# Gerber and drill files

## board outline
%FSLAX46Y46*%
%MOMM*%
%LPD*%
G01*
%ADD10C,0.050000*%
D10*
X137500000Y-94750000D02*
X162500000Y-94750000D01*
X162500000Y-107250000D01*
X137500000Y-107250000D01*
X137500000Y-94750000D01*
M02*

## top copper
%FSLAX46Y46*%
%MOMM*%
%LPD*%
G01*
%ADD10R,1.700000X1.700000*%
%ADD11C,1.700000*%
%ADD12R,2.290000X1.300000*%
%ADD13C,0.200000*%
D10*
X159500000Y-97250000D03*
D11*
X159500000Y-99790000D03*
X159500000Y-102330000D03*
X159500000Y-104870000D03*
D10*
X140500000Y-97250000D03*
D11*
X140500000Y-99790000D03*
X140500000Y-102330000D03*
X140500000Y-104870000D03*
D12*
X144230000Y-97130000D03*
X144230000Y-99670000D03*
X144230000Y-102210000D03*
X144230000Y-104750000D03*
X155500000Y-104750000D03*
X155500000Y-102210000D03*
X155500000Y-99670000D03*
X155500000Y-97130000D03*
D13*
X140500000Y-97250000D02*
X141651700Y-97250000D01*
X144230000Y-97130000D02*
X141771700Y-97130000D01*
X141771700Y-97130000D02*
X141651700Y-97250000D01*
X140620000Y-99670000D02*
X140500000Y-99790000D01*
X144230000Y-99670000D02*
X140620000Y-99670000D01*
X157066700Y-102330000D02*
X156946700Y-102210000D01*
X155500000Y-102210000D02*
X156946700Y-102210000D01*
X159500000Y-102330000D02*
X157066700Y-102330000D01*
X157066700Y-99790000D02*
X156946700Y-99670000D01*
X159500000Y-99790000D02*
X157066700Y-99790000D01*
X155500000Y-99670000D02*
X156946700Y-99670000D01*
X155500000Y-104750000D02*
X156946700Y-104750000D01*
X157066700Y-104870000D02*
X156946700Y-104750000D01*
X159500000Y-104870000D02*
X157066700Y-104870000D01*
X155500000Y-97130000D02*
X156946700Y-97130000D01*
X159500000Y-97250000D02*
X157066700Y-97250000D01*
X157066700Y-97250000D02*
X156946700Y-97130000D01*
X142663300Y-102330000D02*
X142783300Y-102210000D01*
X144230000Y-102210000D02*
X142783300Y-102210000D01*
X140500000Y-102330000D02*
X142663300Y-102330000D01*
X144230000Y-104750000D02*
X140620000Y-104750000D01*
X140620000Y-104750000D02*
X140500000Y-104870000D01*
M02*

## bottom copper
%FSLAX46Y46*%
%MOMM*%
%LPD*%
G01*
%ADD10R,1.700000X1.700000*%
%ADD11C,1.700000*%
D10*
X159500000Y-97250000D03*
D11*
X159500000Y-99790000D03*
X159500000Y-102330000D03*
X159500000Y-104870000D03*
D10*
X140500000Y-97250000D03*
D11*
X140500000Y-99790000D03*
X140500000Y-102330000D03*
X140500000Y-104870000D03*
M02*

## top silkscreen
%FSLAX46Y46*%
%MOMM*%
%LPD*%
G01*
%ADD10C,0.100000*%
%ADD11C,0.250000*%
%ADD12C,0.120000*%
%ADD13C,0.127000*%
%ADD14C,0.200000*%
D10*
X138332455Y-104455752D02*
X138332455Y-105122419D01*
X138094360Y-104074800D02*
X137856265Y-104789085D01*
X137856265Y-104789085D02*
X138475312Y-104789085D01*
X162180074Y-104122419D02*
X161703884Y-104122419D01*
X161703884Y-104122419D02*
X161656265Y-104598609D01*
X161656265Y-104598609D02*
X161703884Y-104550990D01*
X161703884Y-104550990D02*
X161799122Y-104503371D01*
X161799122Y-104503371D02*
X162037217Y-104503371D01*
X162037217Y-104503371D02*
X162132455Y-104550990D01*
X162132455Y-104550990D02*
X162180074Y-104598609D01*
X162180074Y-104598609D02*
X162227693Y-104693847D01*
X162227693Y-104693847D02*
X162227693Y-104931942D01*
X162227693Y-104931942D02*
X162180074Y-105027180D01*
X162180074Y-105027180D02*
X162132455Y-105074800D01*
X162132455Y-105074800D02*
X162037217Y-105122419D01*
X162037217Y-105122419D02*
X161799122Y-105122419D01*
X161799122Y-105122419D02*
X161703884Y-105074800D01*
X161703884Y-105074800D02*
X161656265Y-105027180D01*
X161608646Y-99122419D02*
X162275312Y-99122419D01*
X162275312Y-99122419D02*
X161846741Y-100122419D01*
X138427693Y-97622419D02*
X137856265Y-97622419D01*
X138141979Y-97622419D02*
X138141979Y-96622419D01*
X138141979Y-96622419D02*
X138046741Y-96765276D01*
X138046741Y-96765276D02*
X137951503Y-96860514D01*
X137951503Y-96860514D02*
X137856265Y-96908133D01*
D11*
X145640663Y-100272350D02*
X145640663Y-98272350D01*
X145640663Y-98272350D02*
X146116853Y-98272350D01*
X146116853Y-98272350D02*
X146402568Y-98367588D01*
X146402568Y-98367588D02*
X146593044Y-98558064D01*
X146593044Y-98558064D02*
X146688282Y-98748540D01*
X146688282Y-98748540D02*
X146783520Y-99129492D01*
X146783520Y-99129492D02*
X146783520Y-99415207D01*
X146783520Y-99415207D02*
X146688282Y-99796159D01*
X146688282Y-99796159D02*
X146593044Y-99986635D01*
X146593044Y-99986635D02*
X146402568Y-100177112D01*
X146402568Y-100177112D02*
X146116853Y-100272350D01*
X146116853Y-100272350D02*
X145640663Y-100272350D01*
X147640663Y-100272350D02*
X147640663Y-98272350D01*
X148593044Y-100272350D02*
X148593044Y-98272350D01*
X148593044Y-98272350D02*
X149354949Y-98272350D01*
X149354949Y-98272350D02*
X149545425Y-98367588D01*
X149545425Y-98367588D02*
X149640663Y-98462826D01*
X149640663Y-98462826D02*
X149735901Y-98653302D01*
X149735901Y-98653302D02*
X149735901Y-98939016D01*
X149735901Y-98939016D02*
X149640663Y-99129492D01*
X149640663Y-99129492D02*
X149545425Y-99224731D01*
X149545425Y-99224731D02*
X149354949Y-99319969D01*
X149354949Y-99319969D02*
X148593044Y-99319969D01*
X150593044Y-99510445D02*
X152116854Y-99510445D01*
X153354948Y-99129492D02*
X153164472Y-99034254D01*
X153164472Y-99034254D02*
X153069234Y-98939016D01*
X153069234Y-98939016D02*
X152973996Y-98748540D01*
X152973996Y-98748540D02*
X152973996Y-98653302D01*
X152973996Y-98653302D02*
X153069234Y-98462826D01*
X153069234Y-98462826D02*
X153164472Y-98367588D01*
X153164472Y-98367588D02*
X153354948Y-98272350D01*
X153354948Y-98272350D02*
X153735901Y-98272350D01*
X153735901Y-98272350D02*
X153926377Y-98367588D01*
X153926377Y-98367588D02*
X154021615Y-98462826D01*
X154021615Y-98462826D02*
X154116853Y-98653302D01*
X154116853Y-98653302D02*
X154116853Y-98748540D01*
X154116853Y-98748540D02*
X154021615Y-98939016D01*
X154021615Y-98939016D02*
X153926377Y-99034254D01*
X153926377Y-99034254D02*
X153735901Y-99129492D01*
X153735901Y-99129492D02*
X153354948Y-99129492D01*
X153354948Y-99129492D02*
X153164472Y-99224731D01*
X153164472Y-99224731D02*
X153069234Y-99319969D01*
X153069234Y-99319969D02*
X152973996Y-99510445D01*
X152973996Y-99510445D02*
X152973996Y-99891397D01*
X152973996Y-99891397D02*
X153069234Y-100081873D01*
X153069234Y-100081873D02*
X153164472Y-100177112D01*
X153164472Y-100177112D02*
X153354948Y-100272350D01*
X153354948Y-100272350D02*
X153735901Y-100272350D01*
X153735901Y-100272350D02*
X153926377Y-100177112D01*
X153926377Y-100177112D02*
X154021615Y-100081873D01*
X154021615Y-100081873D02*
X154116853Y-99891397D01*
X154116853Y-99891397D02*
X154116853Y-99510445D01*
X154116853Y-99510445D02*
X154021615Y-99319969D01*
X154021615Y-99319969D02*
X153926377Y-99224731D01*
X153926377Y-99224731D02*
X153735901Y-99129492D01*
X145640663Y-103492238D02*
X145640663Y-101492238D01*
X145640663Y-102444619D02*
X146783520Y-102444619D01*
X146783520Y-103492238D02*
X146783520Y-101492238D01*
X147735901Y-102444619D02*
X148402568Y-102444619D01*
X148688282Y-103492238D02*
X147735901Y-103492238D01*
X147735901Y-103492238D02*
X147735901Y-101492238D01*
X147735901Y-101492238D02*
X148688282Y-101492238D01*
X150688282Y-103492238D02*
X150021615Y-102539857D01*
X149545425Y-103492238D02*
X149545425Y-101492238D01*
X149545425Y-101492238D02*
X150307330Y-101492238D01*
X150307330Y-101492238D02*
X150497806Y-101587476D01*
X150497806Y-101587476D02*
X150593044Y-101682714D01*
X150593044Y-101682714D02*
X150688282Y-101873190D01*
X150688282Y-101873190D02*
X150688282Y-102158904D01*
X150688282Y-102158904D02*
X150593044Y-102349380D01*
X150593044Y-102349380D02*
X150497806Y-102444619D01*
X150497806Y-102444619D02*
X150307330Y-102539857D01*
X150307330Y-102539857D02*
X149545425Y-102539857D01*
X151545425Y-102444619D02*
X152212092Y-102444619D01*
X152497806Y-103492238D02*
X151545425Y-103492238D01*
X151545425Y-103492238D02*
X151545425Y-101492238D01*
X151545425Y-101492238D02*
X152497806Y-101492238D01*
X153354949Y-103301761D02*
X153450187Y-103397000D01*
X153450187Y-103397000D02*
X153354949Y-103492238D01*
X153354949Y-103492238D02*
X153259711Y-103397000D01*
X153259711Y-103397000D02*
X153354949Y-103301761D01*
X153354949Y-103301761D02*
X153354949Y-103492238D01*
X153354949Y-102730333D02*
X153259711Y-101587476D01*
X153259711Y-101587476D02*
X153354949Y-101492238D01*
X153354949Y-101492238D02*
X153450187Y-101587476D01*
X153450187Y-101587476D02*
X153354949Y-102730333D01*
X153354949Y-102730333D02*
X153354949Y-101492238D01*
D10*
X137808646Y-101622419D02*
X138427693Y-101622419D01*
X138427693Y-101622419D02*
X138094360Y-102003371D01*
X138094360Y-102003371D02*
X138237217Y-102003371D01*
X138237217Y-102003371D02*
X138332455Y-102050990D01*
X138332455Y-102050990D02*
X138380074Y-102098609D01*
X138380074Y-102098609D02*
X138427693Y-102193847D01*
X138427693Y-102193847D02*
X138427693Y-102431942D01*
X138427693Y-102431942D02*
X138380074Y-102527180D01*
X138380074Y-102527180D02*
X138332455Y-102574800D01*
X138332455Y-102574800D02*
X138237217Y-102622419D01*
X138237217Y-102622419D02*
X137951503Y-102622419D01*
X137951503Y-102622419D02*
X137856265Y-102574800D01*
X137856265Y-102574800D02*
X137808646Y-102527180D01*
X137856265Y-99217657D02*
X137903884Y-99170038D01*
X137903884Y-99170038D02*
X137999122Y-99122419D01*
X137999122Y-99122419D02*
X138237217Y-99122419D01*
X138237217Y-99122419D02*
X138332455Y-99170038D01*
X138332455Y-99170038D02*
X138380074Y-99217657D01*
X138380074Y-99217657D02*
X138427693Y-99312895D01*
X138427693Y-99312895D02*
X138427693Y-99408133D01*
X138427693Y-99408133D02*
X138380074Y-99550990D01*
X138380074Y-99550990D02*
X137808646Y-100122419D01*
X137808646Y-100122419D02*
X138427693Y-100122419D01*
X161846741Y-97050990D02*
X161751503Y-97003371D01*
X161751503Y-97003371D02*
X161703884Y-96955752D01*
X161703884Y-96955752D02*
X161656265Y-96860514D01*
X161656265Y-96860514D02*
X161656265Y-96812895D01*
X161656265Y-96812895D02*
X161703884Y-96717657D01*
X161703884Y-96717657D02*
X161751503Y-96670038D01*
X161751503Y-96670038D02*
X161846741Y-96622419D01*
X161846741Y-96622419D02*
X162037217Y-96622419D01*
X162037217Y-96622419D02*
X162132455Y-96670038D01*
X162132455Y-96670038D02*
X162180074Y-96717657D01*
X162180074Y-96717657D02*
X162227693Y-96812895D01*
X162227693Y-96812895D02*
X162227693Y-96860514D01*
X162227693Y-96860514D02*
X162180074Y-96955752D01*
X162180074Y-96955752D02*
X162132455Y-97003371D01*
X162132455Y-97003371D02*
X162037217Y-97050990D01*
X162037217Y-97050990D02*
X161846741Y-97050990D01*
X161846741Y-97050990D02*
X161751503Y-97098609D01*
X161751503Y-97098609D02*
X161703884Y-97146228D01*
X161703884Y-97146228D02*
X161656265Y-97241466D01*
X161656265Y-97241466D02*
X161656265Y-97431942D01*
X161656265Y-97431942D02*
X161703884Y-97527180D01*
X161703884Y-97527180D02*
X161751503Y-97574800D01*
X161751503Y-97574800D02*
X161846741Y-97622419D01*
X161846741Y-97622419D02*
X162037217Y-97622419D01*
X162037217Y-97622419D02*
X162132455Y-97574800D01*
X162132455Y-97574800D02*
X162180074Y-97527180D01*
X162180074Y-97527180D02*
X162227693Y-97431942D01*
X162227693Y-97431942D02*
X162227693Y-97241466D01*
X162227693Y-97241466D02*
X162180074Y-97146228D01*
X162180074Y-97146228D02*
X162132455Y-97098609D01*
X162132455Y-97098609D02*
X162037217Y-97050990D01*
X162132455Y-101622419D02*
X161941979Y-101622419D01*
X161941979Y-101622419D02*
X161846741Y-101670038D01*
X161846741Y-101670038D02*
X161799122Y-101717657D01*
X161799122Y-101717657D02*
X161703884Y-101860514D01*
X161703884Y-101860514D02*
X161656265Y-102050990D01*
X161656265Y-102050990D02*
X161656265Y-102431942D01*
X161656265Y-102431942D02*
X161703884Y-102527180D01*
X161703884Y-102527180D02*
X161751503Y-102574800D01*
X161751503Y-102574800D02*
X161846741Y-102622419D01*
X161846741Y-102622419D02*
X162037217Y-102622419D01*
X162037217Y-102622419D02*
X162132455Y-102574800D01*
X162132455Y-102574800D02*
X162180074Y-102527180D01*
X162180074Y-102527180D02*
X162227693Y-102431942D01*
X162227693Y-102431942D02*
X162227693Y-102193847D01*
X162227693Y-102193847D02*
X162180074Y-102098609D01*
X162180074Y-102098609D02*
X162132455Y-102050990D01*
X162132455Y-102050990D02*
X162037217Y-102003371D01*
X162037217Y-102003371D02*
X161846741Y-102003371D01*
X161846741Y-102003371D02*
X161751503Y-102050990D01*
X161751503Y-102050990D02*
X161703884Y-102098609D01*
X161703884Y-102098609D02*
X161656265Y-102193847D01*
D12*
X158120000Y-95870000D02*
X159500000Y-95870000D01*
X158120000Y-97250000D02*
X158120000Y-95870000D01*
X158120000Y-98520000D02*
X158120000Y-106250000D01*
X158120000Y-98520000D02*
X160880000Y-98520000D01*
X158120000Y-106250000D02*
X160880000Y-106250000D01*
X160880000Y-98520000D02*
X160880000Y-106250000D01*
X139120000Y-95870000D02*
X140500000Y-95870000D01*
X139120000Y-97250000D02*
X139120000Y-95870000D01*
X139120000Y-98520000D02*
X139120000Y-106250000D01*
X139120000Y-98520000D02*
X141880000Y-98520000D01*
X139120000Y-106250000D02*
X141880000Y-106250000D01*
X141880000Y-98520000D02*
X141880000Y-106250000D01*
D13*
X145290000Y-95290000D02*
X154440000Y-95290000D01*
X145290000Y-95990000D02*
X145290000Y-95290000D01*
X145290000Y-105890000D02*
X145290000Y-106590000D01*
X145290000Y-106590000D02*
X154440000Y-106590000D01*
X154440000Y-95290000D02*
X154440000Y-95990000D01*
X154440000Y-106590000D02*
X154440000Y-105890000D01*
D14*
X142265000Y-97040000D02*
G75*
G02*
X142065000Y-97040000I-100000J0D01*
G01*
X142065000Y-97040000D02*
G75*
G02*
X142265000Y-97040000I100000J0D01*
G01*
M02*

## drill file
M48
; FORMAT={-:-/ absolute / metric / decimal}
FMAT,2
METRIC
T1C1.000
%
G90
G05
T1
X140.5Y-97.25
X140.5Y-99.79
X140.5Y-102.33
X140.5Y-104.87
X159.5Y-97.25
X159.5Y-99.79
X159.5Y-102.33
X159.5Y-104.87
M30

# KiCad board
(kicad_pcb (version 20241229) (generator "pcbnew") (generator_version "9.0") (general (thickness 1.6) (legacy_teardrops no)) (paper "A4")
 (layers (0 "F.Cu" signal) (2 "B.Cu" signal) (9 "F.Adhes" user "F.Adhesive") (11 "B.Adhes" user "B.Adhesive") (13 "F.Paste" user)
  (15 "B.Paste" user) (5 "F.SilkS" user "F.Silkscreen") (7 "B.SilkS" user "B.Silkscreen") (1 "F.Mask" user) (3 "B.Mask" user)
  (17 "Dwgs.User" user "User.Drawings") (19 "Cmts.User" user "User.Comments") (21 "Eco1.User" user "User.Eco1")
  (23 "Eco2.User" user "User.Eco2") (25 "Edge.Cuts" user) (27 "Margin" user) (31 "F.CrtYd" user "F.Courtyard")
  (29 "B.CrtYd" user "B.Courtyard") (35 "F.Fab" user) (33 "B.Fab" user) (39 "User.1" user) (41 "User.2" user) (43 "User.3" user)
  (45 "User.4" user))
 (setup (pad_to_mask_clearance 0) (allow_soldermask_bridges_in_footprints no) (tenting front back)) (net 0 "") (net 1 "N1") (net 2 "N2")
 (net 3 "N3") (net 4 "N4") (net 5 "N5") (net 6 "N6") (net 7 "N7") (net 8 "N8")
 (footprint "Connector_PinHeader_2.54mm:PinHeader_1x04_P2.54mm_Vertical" (layer "F.Cu") (at 159.5 97.25)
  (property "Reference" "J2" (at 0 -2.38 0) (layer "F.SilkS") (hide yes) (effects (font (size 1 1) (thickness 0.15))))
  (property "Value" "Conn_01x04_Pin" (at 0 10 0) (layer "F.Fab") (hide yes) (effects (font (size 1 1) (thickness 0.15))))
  (fp_line (start -1.38 -1.38) (end 0 -1.38) (stroke (width 0.12) (type solid)) (layer "F.SilkS"))
  (fp_line (start -1.38 0) (end -1.38 -1.38) (stroke (width 0.12) (type solid)) (layer "F.SilkS"))
  (fp_line (start -1.38 1.27) (end -1.38 9) (stroke (width 0.12) (type solid)) (layer "F.SilkS"))
  (fp_line (start -1.38 1.27) (end 1.38 1.27) (stroke (width 0.12) (type solid)) (layer "F.SilkS"))
  (fp_line (start -1.38 9) (end 1.38 9) (stroke (width 0.12) (type solid)) (layer "F.SilkS"))
  (fp_line (start 1.38 1.27) (end 1.38 9) (stroke (width 0.12) (type solid)) (layer "F.SilkS"))
  (pad "1" thru_hole rect (at 0 0) (size 1.7 1.7) (drill 1) (layers "*.Cu" "*.Mask") (remove_unused_layers no) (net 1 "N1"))
  (pad "2" thru_hole circle (at 0 2.54) (size 1.7 1.7) (drill 1) (layers "*.Cu" "*.Mask") (remove_unused_layers no) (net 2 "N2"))
  (pad "3" thru_hole circle (at 0 5.08) (size 1.7 1.7) (drill 1) (layers "*.Cu" "*.Mask") (remove_unused_layers no) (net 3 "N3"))
  (pad "4" thru_hole circle (at 0 7.62) (size 1.7 1.7) (drill 1) (layers "*.Cu" "*.Mask") (remove_unused_layers no) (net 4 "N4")))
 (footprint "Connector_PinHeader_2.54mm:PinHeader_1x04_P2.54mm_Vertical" (layer "F.Cu") (at 140.5 97.25)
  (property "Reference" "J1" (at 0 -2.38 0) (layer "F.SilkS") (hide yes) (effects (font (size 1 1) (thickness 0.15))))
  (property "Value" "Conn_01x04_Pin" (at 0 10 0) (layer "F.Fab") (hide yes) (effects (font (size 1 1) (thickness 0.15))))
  (fp_line (start -1.38 -1.38) (end 0 -1.38) (stroke (width 0.12) (type solid)) (layer "F.SilkS"))
  (fp_line (start -1.38 0) (end -1.38 -1.38) (stroke (width 0.12) (type solid)) (layer "F.SilkS"))
  (fp_line (start -1.38 1.27) (end -1.38 9) (stroke (width 0.12) (type solid)) (layer "F.SilkS"))
  (fp_line (start -1.38 1.27) (end 1.38 1.27) (stroke (width 0.12) (type solid)) (layer "F.SilkS"))
  (fp_line (start -1.38 9) (end 1.38 9) (stroke (width 0.12) (type solid)) (layer "F.SilkS"))
  (fp_line (start 1.38 1.27) (end 1.38 9) (stroke (width 0.12) (type solid)) (layer "F.SilkS"))
  (pad "1" thru_hole rect (at 0 0) (size 1.7 1.7) (drill 1) (layers "*.Cu" "*.Mask") (remove_unused_layers no) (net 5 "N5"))
  (pad "2" thru_hole circle (at 0 2.54) (size 1.7 1.7) (drill 1) (layers "*.Cu" "*.Mask") (remove_unused_layers no) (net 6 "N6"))
  (pad "3" thru_hole circle (at 0 5.08) (size 1.7 1.7) (drill 1) (layers "*.Cu" "*.Mask") (remove_unused_layers no) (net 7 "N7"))
  (pad "4" thru_hole circle (at 0 7.62) (size 1.7 1.7) (drill 1) (layers "*.Cu" "*.Mask") (remove_unused_layers no) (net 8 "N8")))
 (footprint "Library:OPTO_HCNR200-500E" (layer "F.Cu") (at 149.865 100.94)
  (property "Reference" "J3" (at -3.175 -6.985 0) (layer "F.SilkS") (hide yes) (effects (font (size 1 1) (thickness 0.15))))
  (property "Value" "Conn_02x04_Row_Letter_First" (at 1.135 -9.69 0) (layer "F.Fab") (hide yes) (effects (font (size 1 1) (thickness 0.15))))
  (fp_line (start -4.575 -5.65) (end 4.575 -5.65) (stroke (width 0.127) (type solid)) (layer "F.SilkS"))
  (fp_line (start -4.575 -4.95) (end -4.575 -5.65) (stroke (width 0.127) (type solid)) (layer "F.SilkS"))
  (fp_line (start -4.575 4.95) (end -4.575 5.65) (stroke (width 0.127) (type solid)) (layer "F.SilkS"))
  (fp_line (start -4.575 5.65) (end 4.575 5.65) (stroke (width 0.127) (type solid)) (layer "F.SilkS"))
  (fp_line (start 4.575 -5.65) (end 4.575 -4.95) (stroke (width 0.127) (type solid)) (layer "F.SilkS"))
  (fp_line (start 4.575 5.65) (end 4.575 4.95) (stroke (width 0.127) (type solid)) (layer "F.SilkS"))
  (fp_circle (center -7.7 -3.9) (end -7.6 -3.9) (stroke (width 0.2) (type solid)) (fill no) (layer "F.SilkS"))
  (pad "1" smd rect (at -5.635 -3.81) (size 2.29 1.3) (layers "F.Cu" "F.Mask" "F.Paste") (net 5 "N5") (solder_mask_margin 0.102))
  (pad "2" smd rect (at -5.635 -1.27) (size 2.29 1.3) (layers "F.Cu" "F.Mask" "F.Paste") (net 6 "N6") (solder_mask_margin 0.102))
  (pad "3" smd rect (at -5.635 1.27) (size 2.29 1.3) (layers "F.Cu" "F.Mask" "F.Paste") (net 7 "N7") (solder_mask_margin 0.102))
  (pad "4" smd rect (at -5.635 3.81) (size 2.29 1.3) (layers "F.Cu" "F.Mask" "F.Paste") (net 8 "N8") (solder_mask_margin 0.102))
  (pad "5" smd rect (at 5.635 3.81) (size 2.29 1.3) (layers "F.Cu" "F.Mask" "F.Paste") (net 4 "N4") (solder_mask_margin 0.102))
  (pad "6" smd rect (at 5.635 1.27) (size 2.29 1.3) (layers "F.Cu" "F.Mask" "F.Paste") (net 3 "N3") (solder_mask_margin 0.102))
  (pad "7" smd rect (at 5.635 -1.27) (size 2.29 1.3) (layers "F.Cu" "F.Mask" "F.Paste") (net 2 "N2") (solder_mask_margin 0.102))
  (pad "8" smd rect (at 5.635 -3.81) (size 2.29 1.3) (layers "F.Cu" "F.Mask" "F.Paste") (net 1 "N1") (solder_mask_margin 0.102)))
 (gr_rect (start 137.5 94.75) (end 162.5 107.25) (stroke (width 0.05) (type default)) (fill no) (layer "Edge.Cuts"))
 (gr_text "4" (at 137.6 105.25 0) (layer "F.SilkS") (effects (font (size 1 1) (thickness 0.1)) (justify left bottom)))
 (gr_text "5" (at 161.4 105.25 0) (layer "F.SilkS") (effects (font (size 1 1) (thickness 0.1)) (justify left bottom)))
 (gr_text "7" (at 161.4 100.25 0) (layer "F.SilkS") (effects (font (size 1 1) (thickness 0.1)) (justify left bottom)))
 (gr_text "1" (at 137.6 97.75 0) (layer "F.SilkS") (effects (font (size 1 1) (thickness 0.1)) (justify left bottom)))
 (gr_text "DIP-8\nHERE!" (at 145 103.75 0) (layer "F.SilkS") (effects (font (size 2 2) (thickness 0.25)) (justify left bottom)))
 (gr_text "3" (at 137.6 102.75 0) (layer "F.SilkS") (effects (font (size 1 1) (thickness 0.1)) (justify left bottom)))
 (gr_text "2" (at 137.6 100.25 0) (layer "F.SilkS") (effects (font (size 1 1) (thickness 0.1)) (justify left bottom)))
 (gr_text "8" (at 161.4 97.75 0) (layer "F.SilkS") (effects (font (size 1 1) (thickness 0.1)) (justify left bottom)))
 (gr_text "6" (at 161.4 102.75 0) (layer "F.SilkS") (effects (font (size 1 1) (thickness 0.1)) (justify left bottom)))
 (segment (start 140.5 97.25) (end 141.6517 97.25) (width 0.2) (layer "F.Cu") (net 5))
 (segment (start 144.23 97.13) (end 141.7717 97.13) (width 0.2) (layer "F.Cu") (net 5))
 (segment (start 141.7717 97.13) (end 141.6517 97.25) (width 0.2) (layer "F.Cu") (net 5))
 (segment (start 140.62 99.67) (end 140.5 99.79) (width 0.2) (layer "F.Cu") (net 6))
 (segment (start 144.23 99.67) (end 140.62 99.67) (width 0.2) (layer "F.Cu") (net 6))
 (segment (start 157.0667 102.33) (end 156.9467 102.21) (width 0.2) (layer "F.Cu") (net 3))
 (segment (start 155.5 102.21) (end 156.9467 102.21) (width 0.2) (layer "F.Cu") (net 3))
 (segment (start 159.5 102.33) (end 157.0667 102.33) (width 0.2) (layer "F.Cu") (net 3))
 (segment (start 157.0667 99.79) (end 156.9467 99.67) (width 0.2) (layer "F.Cu") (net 2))
 (segment (start 159.5 99.79) (end 157.0667 99.79) (width 0.2) (layer "F.Cu") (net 2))
 (segment (start 155.5 99.67) (end 156.9467 99.67) (width 0.2) (layer "F.Cu") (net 2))
 (segment (start 155.5 104.75) (end 156.9467 104.75) (width 0.2) (layer "F.Cu") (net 4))
 (segment (start 157.0667 104.87) (end 156.9467 104.75) (width 0.2) (layer "F.Cu") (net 4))
 (segment (start 159.5 104.87) (end 157.0667 104.87) (width 0.2) (layer "F.Cu") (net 4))
 (segment (start 155.5 97.13) (end 156.9467 97.13) (width 0.2) (layer "F.Cu") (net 1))
 (segment (start 159.5 97.25) (end 157.0667 97.25) (width 0.2) (layer "F.Cu") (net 1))
 (segment (start 157.0667 97.25) (end 156.9467 97.13) (width 0.2) (layer "F.Cu") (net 1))
 (segment (start 142.6633 102.33) (end 142.7833 102.21) (width 0.2) (layer "F.Cu") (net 7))
 (segment (start 144.23 102.21) (end 142.7833 102.21) (width 0.2) (layer "F.Cu") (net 7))
 (segment (start 140.5 102.33) (end 142.6633 102.33) (width 0.2) (layer "F.Cu") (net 7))
 (segment (start 144.23 104.75) (end 140.62 104.75) (width 0.2) (layer "F.Cu") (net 8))
 (segment (start 140.62 104.75) (end 140.5 104.87) (width 0.2) (layer "F.Cu") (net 8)))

